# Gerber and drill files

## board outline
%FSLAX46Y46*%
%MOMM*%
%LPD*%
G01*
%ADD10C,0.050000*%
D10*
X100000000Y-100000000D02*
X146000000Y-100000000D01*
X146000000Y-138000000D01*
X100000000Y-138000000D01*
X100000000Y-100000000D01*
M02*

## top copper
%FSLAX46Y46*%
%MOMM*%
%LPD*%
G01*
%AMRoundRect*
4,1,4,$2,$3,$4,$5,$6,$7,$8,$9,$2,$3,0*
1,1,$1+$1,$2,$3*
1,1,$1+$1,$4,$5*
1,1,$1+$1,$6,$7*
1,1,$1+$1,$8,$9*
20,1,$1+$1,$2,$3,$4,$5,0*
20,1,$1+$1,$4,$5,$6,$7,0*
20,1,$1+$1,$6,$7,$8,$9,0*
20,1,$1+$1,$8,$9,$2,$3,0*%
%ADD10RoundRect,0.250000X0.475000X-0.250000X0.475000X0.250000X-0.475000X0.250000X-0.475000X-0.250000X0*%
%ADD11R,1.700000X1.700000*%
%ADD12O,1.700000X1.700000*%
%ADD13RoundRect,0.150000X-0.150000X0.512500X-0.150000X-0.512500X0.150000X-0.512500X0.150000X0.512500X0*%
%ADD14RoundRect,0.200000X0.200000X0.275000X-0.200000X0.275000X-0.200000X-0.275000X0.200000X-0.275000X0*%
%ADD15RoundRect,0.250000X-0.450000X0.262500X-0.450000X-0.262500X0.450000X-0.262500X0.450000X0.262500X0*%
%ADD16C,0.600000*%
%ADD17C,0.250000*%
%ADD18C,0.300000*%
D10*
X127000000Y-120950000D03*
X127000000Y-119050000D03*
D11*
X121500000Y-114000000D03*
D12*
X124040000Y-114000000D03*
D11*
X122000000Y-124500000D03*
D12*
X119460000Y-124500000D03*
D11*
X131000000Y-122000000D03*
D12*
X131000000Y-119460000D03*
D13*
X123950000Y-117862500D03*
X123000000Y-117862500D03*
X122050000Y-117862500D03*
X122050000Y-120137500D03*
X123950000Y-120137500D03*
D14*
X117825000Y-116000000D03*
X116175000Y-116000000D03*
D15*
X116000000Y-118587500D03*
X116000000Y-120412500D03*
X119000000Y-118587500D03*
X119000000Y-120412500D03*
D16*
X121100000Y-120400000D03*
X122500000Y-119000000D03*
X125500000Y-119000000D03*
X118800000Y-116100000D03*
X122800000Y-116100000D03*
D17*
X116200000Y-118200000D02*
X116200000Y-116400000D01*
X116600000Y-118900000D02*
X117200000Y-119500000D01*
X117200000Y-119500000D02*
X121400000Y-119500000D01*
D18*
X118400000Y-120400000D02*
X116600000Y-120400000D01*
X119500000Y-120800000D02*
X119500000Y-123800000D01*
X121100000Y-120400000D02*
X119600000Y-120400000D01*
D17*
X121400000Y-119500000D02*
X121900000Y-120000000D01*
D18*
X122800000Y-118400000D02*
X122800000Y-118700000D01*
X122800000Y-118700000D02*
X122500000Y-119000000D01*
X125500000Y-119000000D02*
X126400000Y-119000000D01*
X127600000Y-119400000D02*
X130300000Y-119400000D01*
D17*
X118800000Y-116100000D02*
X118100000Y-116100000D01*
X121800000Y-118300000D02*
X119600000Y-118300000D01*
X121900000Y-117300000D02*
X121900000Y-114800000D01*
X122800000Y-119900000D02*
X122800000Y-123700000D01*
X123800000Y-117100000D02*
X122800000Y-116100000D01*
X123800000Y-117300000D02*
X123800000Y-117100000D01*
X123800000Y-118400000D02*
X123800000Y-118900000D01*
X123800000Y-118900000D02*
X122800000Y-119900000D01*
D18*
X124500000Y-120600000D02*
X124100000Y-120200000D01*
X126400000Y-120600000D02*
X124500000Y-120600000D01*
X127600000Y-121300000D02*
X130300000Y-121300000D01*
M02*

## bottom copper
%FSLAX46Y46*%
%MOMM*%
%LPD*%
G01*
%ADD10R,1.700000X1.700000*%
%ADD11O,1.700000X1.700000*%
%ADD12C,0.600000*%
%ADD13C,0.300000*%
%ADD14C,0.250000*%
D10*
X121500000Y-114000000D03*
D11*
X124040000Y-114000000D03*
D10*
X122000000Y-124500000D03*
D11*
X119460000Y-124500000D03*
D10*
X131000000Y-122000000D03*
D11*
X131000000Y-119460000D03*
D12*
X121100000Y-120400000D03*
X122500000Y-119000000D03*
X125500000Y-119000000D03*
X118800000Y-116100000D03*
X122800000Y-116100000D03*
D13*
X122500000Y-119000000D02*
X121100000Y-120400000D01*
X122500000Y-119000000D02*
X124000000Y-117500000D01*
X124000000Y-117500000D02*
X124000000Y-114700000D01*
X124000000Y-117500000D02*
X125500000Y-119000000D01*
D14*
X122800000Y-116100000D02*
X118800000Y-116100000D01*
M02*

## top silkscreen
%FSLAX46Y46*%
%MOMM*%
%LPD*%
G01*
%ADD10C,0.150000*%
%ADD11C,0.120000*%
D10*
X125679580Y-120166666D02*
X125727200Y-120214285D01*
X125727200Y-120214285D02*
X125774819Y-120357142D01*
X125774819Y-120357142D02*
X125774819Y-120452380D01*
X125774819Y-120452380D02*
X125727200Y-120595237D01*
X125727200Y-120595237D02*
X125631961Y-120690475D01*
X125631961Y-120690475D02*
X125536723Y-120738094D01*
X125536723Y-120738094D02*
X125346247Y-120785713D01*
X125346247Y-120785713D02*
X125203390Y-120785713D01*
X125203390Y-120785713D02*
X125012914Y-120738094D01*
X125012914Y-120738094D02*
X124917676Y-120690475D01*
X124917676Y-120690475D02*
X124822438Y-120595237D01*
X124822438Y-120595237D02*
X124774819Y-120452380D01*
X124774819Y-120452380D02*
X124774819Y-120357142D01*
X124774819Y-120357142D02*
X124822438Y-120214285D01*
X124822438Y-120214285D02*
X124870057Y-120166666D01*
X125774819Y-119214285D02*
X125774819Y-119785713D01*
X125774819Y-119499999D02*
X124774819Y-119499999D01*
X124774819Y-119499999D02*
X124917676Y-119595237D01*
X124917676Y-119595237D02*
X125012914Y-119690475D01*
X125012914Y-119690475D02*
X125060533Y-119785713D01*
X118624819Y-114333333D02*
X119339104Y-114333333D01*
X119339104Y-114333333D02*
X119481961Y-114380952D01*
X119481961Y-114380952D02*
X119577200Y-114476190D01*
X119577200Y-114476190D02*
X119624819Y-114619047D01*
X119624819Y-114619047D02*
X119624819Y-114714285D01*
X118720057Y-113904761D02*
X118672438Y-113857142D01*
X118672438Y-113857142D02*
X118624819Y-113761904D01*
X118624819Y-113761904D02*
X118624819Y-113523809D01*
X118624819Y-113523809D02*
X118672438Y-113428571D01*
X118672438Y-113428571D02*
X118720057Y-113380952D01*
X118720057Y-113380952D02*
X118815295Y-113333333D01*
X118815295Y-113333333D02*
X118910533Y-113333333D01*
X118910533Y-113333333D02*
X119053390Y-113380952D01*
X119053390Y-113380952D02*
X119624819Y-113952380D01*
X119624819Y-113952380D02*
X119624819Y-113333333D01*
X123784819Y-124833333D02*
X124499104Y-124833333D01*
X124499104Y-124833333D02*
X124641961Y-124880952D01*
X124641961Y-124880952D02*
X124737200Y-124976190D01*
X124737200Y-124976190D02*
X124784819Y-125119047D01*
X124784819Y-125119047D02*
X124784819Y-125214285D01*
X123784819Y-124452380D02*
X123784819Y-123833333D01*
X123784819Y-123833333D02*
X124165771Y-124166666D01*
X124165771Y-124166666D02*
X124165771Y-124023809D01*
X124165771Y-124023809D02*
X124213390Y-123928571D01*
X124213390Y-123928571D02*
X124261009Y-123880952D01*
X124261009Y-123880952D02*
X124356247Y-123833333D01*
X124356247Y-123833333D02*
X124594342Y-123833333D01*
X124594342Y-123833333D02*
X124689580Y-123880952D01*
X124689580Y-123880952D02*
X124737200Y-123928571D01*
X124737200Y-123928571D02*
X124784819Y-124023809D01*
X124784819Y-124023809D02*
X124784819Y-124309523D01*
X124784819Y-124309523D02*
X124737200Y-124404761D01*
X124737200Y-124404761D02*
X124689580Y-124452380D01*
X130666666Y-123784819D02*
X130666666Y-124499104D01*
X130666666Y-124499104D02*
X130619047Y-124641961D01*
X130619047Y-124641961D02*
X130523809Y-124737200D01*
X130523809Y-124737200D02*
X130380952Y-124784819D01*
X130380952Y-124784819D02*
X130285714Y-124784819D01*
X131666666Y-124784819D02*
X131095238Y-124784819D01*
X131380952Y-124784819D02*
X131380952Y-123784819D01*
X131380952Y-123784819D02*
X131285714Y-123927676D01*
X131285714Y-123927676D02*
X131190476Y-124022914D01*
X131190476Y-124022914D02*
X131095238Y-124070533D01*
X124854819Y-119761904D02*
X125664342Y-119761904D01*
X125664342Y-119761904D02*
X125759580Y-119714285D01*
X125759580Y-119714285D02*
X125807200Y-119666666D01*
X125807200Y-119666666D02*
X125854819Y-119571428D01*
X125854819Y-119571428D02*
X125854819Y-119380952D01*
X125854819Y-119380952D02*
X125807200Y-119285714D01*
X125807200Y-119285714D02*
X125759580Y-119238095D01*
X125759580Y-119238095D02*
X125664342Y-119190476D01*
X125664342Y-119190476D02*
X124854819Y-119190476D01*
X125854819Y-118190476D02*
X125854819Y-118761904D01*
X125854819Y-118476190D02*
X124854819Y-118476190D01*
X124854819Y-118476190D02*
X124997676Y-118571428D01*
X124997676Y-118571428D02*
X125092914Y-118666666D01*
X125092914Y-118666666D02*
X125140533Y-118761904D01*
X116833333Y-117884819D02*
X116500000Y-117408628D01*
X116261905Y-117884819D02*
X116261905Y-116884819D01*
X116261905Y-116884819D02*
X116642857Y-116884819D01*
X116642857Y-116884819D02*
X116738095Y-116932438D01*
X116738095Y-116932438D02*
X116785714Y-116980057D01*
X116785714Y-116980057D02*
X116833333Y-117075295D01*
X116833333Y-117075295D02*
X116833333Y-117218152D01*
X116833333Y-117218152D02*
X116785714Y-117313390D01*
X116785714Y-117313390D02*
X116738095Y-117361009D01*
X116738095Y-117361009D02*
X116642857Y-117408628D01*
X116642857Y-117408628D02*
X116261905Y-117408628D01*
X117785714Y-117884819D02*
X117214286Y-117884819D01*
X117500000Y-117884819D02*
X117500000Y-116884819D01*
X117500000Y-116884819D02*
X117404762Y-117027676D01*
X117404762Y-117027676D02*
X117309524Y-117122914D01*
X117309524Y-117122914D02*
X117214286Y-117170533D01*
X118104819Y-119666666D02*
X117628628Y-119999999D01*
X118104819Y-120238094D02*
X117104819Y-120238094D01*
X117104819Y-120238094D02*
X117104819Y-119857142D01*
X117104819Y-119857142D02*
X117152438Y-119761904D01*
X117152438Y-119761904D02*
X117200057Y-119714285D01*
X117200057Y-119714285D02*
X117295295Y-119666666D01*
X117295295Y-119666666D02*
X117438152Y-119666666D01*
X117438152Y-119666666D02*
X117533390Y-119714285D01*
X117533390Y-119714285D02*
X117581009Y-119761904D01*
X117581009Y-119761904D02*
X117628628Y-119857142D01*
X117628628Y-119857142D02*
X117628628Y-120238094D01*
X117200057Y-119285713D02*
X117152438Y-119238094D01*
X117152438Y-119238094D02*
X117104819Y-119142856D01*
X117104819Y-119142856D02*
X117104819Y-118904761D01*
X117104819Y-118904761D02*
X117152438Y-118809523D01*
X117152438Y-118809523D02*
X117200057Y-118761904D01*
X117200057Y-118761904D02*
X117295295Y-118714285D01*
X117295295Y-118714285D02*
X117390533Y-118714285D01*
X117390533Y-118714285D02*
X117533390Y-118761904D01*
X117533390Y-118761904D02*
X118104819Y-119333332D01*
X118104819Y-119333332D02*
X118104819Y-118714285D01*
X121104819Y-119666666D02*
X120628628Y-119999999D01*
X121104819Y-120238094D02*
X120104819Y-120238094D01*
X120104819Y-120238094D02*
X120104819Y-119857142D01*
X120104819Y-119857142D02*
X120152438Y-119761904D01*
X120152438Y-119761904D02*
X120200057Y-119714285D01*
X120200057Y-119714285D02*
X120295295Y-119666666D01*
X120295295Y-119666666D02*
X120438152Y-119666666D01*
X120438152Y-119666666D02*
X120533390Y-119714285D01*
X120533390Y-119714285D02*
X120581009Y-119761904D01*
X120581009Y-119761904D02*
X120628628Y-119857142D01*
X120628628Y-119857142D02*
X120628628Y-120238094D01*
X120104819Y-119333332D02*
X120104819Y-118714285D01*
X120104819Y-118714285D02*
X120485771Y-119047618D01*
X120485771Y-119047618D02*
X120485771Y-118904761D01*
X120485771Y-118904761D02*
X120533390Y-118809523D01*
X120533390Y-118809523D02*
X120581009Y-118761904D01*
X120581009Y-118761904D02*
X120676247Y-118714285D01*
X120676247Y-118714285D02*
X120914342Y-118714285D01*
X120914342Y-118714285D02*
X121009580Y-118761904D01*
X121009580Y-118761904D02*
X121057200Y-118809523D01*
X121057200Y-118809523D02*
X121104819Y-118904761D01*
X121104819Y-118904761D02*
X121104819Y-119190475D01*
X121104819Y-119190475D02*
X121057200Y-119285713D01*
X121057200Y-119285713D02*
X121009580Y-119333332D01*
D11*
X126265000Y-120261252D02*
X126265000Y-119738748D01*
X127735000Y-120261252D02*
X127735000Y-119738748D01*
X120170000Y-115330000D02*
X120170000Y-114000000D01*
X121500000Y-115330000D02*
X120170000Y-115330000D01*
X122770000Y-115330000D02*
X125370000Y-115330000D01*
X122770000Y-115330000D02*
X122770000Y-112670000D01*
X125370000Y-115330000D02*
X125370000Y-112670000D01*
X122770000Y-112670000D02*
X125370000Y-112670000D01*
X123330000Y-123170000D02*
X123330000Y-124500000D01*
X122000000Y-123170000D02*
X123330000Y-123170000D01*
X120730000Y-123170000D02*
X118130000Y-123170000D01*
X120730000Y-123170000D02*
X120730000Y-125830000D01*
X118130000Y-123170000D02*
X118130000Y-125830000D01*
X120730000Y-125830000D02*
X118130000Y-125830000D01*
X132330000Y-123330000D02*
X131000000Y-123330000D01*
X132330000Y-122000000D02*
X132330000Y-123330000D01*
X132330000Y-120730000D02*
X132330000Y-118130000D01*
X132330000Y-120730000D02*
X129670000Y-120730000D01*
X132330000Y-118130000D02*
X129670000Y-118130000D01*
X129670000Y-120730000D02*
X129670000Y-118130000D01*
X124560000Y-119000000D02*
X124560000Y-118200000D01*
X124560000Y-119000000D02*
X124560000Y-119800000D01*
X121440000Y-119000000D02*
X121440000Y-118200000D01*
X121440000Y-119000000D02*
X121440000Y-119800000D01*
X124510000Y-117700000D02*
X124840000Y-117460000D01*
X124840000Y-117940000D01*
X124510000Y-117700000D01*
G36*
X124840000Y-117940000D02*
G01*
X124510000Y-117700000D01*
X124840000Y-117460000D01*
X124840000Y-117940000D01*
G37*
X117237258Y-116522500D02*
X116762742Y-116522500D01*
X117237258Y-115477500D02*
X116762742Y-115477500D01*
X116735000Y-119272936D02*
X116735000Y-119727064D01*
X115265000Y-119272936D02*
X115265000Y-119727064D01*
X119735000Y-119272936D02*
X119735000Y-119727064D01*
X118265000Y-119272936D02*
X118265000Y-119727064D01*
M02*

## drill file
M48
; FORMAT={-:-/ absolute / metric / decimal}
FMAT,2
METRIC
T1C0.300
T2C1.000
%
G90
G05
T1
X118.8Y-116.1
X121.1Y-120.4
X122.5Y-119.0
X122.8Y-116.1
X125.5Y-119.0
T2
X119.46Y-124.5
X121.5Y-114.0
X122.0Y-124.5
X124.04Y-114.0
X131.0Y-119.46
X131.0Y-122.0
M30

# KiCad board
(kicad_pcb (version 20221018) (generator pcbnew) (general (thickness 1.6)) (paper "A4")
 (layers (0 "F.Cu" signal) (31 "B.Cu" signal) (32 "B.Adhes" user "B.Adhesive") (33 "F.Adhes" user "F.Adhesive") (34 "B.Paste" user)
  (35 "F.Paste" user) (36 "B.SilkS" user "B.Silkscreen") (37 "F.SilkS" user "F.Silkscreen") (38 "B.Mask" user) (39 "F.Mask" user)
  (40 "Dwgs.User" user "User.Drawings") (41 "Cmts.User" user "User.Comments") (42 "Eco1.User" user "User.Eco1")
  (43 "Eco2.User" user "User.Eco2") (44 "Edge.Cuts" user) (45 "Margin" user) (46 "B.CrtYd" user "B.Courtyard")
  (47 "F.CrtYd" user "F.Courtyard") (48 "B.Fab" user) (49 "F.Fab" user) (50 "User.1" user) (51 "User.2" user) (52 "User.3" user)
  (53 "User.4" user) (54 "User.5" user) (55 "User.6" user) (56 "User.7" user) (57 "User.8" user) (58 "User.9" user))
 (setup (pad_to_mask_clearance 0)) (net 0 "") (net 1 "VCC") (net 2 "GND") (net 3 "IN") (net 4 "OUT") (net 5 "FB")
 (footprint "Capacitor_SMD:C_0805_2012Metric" (layer "F.Cu") (at 127 120 90)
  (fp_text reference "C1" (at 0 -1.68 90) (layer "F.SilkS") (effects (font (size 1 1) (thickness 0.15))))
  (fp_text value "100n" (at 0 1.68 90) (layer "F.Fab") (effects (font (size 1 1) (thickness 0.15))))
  (fp_line (start -0.261252 -0.735) (end 0.261252 -0.735) (stroke (width 0.12) (type solid)) (layer "F.SilkS"))
  (fp_line (start -0.261252 0.735) (end 0.261252 0.735) (stroke (width 0.12) (type solid)) (layer "F.SilkS"))
  (pad "1" smd roundrect (at -0.95 0 90) (size 1 1.45) (layers "F.Cu" "F.Paste" "F.Mask") (roundrect_rratio 0.25) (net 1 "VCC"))
  (pad "2" smd roundrect (at 0.95 0 90) (size 1 1.45) (layers "F.Cu" "F.Paste" "F.Mask") (roundrect_rratio 0.25) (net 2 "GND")))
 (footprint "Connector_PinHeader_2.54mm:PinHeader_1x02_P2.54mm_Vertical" (layer "F.Cu") (at 121.5 114 90)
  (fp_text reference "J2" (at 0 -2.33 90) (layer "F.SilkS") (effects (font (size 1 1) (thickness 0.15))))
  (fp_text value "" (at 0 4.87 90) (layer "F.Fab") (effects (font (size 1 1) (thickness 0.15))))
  (fp_line (start -1.33 -1.33) (end 0 -1.33) (stroke (width 0.12) (type solid)) (layer "F.SilkS"))
  (fp_line (start -1.33 0) (end -1.33 -1.33) (stroke (width 0.12) (type solid)) (layer "F.SilkS"))
  (fp_line (start -1.33 1.27) (end -1.33 3.87) (stroke (width 0.12) (type solid)) (layer "F.SilkS"))
  (fp_line (start -1.33 1.27) (end 1.33 1.27) (stroke (width 0.12) (type solid)) (layer "F.SilkS"))
  (fp_line (start -1.33 3.87) (end 1.33 3.87) (stroke (width 0.12) (type solid)) (layer "F.SilkS"))
  (fp_line (start 1.33 1.27) (end 1.33 3.87) (stroke (width 0.12) (type solid)) (layer "F.SilkS"))
  (pad "1" thru_hole rect (at 0 0 90) (size 1.7 1.7) (drill 1) (layers "*.Cu" "*.Mask") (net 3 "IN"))
  (pad "2" thru_hole oval (at 0 2.54 90) (size 1.7 1.7) (drill 1) (layers "*.Cu" "*.Mask") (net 2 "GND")))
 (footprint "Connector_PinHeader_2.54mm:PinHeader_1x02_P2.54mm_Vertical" (layer "F.Cu") (at 122 124.5 -90)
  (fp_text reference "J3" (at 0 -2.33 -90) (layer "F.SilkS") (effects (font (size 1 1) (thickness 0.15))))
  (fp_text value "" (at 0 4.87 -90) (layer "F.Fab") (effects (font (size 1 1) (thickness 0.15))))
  (fp_line (start -1.33 -1.33) (end 0 -1.33) (stroke (width 0.12) (type solid)) (layer "F.SilkS"))
  (fp_line (start -1.33 0) (end -1.33 -1.33) (stroke (width 0.12) (type solid)) (layer "F.SilkS"))
  (fp_line (start -1.33 1.27) (end -1.33 3.87) (stroke (width 0.12) (type solid)) (layer "F.SilkS"))
  (fp_line (start -1.33 1.27) (end 1.33 1.27) (stroke (width 0.12) (type solid)) (layer "F.SilkS"))
  (fp_line (start -1.33 3.87) (end 1.33 3.87) (stroke (width 0.12) (type solid)) (layer "F.SilkS"))
  (fp_line (start 1.33 1.27) (end 1.33 3.87) (stroke (width 0.12) (type solid)) (layer "F.SilkS"))
  (pad "1" thru_hole rect (at 0 0 270) (size 1.7 1.7) (drill 1) (layers "*.Cu" "*.Mask") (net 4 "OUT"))
  (pad "2" thru_hole oval (at 0 2.54 270) (size 1.7 1.7) (drill 1) (layers "*.Cu" "*.Mask") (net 2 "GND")))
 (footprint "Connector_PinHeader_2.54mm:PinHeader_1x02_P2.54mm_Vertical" (layer "F.Cu") (at 131 122 180)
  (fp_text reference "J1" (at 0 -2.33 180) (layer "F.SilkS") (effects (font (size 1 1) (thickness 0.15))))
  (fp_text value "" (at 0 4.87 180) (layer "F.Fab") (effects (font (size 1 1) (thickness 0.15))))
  (fp_line (start -1.33 -1.33) (end 0 -1.33) (stroke (width 0.12) (type solid)) (layer "F.SilkS"))
  (fp_line (start -1.33 0) (end -1.33 -1.33) (stroke (width 0.12) (type solid)) (layer "F.SilkS"))
  (fp_line (start -1.33 1.27) (end -1.33 3.87) (stroke (width 0.12) (type solid)) (layer "F.SilkS"))
  (fp_line (start -1.33 1.27) (end 1.33 1.27) (stroke (width 0.12) (type solid)) (layer "F.SilkS"))
  (fp_line (start -1.33 3.87) (end 1.33 3.87) (stroke (width 0.12) (type solid)) (layer "F.SilkS"))
  (fp_line (start 1.33 1.27) (end 1.33 3.87) (stroke (width 0.12) (type solid)) (layer "F.SilkS"))
  (pad "1" thru_hole rect (at 0 0 180) (size 1.7 1.7) (drill 1) (layers "*.Cu" "*.Mask") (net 1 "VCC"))
  (pad "2" thru_hole oval (at 0 2.54 180) (size 1.7 1.7) (drill 1) (layers "*.Cu" "*.Mask") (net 2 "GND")))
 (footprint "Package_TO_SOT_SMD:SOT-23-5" (layer "F.Cu") (at 123 119 -90)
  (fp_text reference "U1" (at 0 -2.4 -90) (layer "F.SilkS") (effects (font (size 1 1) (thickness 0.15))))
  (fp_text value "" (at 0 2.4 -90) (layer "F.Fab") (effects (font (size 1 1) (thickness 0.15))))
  (fp_line (start 0 -1.56) (end -0.8 -1.56) (stroke (width 0.12) (type solid)) (layer "F.SilkS"))
  (fp_line (start 0 -1.56) (end 0.8 -1.56) (stroke (width 0.12) (type solid)) (layer "F.SilkS"))
  (fp_line (start 0 1.56) (end -0.8 1.56) (stroke (width 0.12) (type solid)) (layer "F.SilkS"))
  (fp_line (start 0 1.56) (end 0.8 1.56) (stroke (width 0.12) (type solid)) (layer "F.SilkS"))
  (fp_poly
   (pts (xy -1.3 -1.51) (xy -1.54 -1.84) (xy -1.06 -1.84) (xy -1.3 -1.51)) (stroke (width 0.12) (type solid)) (fill solid) (layer "F.SilkS"))
  (pad "1" smd roundrect (at -1.1375 -0.95 270) (size 1.325 0.6) (layers "F.Cu" "F.Paste" "F.Mask") (roundrect_rratio 0.25) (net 4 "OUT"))
  (pad "2" smd roundrect (at -1.1375 0 270) (size 1.325 0.6) (layers "F.Cu" "F.Paste" "F.Mask") (roundrect_rratio 0.25) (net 2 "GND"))
  (pad "3" smd roundrect (at -1.1375 0.95 270) (size 1.325 0.6) (layers "F.Cu" "F.Paste" "F.Mask") (roundrect_rratio 0.25) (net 3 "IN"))
  (pad "4" smd roundrect (at 1.1375 0.95 270) (size 1.325 0.6) (layers "F.Cu" "F.Paste" "F.Mask") (roundrect_rratio 0.25) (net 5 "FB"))
  (pad "5" smd roundrect (at 1.1375 -0.95 270) (size 1.325 0.6) (layers "F.Cu" "F.Paste" "F.Mask") (roundrect_rratio 0.25) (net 1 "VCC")))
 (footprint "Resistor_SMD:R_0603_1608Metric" (layer "F.Cu") (at 117 116 180)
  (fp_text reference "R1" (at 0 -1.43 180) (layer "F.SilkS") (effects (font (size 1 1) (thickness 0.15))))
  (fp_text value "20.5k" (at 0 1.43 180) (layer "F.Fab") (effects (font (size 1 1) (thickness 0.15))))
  (fp_line (start -0.237258 -0.5225) (end 0.237258 -0.5225) (stroke (width 0.12) (type solid)) (layer "F.SilkS"))
  (fp_line (start -0.237258 0.5225) (end 0.237258 0.5225) (stroke (width 0.12) (type solid)) (layer "F.SilkS"))
  (pad "1" smd roundrect (at -0.825 0 180) (size 0.8 0.95) (layers "F.Cu" "F.Paste" "F.Mask") (roundrect_rratio 0.25) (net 4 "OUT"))
  (pad "2" smd roundrect (at 0.825 0 180) (size 0.8 0.95) (layers "F.Cu" "F.Paste" "F.Mask") (roundrect_rratio 0.25) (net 5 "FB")))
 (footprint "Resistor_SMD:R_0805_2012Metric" (layer "F.Cu") (at 116 119.5 -90)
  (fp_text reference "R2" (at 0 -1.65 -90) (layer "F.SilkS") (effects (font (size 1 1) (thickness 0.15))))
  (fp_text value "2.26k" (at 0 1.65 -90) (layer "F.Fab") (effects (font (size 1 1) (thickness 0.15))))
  (fp_line (start -0.227064 -0.735) (end 0.227064 -0.735) (stroke (width 0.12) (type solid)) (layer "F.SilkS"))
  (fp_line (start -0.227064 0.735) (end 0.227064 0.735) (stroke (width 0.12) (type solid)) (layer "F.SilkS"))
  (pad "1" smd roundrect (at -0.9125 0 270) (size 1.025 1.4) (layers "F.Cu" "F.Paste" "F.Mask") (roundrect_rratio 0.243902) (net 5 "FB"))
  (pad "2" smd roundrect (at 0.9125 0 270) (size 1.025 1.4) (layers "F.Cu" "F.Paste" "F.Mask") (roundrect_rratio 0.243902) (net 2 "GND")))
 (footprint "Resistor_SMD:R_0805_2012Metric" (layer "F.Cu") (at 119 119.5 -90)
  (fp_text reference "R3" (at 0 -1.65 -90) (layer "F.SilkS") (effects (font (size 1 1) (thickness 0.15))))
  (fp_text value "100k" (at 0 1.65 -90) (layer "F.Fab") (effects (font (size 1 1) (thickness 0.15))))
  (fp_line (start -0.227064 -0.735) (end 0.227064 -0.735) (stroke (width 0.12) (type solid)) (layer "F.SilkS"))
  (fp_line (start -0.227064 0.735) (end 0.227064 0.735) (stroke (width 0.12) (type solid)) (layer "F.SilkS"))
  (pad "1" smd roundrect (at -0.9125 0 270) (size 1.025 1.4) (layers "F.Cu" "F.Paste" "F.Mask") (roundrect_rratio 0.243902) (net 3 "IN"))
  (pad "2" smd roundrect (at 0.9125 0 270) (size 1.025 1.4) (layers "F.Cu" "F.Paste" "F.Mask") (roundrect_rratio 0.243902) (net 2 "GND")))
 (gr_rect (start 100 100) (end 146 138) (stroke (width 0.05) (type default)) (fill none) (layer "Edge.Cuts"))
 (segment (start 116.2 118.2) (end 116.2 116.4) (width 0.25) (layer "F.Cu") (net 5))
 (segment (start 116.6 118.9) (end 117.2 119.5) (width 0.25) (layer "F.Cu") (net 5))
 (segment (start 117.2 119.5) (end 121.4 119.5) (width 0.25) (layer "F.Cu") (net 5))
 (segment (start 118.4 120.4) (end 116.6 120.4) (width 0.3) (layer "F.Cu") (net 2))
 (segment (start 119.5 120.8) (end 119.5 123.8) (width 0.3) (layer "F.Cu") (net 2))
 (segment (start 121.1 120.4) (end 119.6 120.4) (width 0.3) (layer "F.Cu") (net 2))
 (segment (start 121.4 119.5) (end 121.9 120) (width 0.25) (layer "F.Cu") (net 5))
 (segment (start 122.8 118.4) (end 122.8 118.7) (width 0.3) (layer "F.Cu") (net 2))
 (segment (start 122.8 118.7) (end 122.5 119) (width 0.3) (layer "F.Cu") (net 2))
 (segment (start 125.5 119) (end 126.4 119) (width 0.3) (layer "F.Cu") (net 2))
 (segment (start 127.6 119.4) (end 130.3 119.4) (width 0.3) (layer "F.Cu") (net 2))
 (via (at 121.1 120.4) (size 0.6) (drill 0.3) (layers "F.Cu" "B.Cu") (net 2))
 (via (at 122.5 119) (size 0.6) (drill 0.3) (layers "F.Cu" "B.Cu") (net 2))
 (via (at 125.5 119) (size 0.6) (drill 0.3) (layers "F.Cu" "B.Cu") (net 2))
 (segment (start 118.8 116.1) (end 118.1 116.1) (width 0.25) (layer "F.Cu") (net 4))
 (segment (start 121.8 118.3) (end 119.6 118.3) (width 0.25) (layer "F.Cu") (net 3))
 (segment (start 121.9 117.3) (end 121.9 114.8) (width 0.25) (layer "F.Cu") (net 3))
 (segment (start 122.5 119) (end 121.1 120.4) (width 0.3) (layer "B.Cu") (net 2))
 (segment (start 122.5 119) (end 124 117.5) (width 0.3) (layer "B.Cu") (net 2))
 (segment (start 122.8 119.9) (end 122.8 123.7) (width 0.25) (layer "F.Cu") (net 4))
 (segment (start 123.8 117.1) (end 122.8 116.1) (width 0.25) (layer "F.Cu") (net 4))
 (segment (start 123.8 117.3) (end 123.8 117.1) (width 0.25) (layer "F.Cu") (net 4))
 (segment (start 123.8 118.4) (end 123.8 118.9) (width 0.25) (layer "F.Cu") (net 4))
 (segment (start 123.8 118.9) (end 122.8 119.9) (width 0.25) (layer "F.Cu") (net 4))
 (segment (start 124 117.5) (end 124 114.7) (width 0.3) (layer "B.Cu") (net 2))
 (segment (start 124 117.5) (end 125.5 119) (width 0.3) (layer "B.Cu") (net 2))
 (via (at 118.8 116.1) (size 0.6) (drill 0.3) (layers "F.Cu" "B.Cu") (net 4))
 (via (at 122.8 116.1) (size 0.6) (drill 0.3) (layers "F.Cu" "B.Cu") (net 4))
 (segment (start 122.8 116.1) (end 118.8 116.1) (width 0.25) (layer "B.Cu") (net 4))
 (segment (start 124.5 120.6) (end 124.1 120.2) (width 0.3) (layer "F.Cu") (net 1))
 (segment (start 126.4 120.6) (end 124.5 120.6) (width 0.3) (layer "F.Cu") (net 1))
 (segment (start 127.6 121.3) (end 130.3 121.3) (width 0.3) (layer "F.Cu") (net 1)))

